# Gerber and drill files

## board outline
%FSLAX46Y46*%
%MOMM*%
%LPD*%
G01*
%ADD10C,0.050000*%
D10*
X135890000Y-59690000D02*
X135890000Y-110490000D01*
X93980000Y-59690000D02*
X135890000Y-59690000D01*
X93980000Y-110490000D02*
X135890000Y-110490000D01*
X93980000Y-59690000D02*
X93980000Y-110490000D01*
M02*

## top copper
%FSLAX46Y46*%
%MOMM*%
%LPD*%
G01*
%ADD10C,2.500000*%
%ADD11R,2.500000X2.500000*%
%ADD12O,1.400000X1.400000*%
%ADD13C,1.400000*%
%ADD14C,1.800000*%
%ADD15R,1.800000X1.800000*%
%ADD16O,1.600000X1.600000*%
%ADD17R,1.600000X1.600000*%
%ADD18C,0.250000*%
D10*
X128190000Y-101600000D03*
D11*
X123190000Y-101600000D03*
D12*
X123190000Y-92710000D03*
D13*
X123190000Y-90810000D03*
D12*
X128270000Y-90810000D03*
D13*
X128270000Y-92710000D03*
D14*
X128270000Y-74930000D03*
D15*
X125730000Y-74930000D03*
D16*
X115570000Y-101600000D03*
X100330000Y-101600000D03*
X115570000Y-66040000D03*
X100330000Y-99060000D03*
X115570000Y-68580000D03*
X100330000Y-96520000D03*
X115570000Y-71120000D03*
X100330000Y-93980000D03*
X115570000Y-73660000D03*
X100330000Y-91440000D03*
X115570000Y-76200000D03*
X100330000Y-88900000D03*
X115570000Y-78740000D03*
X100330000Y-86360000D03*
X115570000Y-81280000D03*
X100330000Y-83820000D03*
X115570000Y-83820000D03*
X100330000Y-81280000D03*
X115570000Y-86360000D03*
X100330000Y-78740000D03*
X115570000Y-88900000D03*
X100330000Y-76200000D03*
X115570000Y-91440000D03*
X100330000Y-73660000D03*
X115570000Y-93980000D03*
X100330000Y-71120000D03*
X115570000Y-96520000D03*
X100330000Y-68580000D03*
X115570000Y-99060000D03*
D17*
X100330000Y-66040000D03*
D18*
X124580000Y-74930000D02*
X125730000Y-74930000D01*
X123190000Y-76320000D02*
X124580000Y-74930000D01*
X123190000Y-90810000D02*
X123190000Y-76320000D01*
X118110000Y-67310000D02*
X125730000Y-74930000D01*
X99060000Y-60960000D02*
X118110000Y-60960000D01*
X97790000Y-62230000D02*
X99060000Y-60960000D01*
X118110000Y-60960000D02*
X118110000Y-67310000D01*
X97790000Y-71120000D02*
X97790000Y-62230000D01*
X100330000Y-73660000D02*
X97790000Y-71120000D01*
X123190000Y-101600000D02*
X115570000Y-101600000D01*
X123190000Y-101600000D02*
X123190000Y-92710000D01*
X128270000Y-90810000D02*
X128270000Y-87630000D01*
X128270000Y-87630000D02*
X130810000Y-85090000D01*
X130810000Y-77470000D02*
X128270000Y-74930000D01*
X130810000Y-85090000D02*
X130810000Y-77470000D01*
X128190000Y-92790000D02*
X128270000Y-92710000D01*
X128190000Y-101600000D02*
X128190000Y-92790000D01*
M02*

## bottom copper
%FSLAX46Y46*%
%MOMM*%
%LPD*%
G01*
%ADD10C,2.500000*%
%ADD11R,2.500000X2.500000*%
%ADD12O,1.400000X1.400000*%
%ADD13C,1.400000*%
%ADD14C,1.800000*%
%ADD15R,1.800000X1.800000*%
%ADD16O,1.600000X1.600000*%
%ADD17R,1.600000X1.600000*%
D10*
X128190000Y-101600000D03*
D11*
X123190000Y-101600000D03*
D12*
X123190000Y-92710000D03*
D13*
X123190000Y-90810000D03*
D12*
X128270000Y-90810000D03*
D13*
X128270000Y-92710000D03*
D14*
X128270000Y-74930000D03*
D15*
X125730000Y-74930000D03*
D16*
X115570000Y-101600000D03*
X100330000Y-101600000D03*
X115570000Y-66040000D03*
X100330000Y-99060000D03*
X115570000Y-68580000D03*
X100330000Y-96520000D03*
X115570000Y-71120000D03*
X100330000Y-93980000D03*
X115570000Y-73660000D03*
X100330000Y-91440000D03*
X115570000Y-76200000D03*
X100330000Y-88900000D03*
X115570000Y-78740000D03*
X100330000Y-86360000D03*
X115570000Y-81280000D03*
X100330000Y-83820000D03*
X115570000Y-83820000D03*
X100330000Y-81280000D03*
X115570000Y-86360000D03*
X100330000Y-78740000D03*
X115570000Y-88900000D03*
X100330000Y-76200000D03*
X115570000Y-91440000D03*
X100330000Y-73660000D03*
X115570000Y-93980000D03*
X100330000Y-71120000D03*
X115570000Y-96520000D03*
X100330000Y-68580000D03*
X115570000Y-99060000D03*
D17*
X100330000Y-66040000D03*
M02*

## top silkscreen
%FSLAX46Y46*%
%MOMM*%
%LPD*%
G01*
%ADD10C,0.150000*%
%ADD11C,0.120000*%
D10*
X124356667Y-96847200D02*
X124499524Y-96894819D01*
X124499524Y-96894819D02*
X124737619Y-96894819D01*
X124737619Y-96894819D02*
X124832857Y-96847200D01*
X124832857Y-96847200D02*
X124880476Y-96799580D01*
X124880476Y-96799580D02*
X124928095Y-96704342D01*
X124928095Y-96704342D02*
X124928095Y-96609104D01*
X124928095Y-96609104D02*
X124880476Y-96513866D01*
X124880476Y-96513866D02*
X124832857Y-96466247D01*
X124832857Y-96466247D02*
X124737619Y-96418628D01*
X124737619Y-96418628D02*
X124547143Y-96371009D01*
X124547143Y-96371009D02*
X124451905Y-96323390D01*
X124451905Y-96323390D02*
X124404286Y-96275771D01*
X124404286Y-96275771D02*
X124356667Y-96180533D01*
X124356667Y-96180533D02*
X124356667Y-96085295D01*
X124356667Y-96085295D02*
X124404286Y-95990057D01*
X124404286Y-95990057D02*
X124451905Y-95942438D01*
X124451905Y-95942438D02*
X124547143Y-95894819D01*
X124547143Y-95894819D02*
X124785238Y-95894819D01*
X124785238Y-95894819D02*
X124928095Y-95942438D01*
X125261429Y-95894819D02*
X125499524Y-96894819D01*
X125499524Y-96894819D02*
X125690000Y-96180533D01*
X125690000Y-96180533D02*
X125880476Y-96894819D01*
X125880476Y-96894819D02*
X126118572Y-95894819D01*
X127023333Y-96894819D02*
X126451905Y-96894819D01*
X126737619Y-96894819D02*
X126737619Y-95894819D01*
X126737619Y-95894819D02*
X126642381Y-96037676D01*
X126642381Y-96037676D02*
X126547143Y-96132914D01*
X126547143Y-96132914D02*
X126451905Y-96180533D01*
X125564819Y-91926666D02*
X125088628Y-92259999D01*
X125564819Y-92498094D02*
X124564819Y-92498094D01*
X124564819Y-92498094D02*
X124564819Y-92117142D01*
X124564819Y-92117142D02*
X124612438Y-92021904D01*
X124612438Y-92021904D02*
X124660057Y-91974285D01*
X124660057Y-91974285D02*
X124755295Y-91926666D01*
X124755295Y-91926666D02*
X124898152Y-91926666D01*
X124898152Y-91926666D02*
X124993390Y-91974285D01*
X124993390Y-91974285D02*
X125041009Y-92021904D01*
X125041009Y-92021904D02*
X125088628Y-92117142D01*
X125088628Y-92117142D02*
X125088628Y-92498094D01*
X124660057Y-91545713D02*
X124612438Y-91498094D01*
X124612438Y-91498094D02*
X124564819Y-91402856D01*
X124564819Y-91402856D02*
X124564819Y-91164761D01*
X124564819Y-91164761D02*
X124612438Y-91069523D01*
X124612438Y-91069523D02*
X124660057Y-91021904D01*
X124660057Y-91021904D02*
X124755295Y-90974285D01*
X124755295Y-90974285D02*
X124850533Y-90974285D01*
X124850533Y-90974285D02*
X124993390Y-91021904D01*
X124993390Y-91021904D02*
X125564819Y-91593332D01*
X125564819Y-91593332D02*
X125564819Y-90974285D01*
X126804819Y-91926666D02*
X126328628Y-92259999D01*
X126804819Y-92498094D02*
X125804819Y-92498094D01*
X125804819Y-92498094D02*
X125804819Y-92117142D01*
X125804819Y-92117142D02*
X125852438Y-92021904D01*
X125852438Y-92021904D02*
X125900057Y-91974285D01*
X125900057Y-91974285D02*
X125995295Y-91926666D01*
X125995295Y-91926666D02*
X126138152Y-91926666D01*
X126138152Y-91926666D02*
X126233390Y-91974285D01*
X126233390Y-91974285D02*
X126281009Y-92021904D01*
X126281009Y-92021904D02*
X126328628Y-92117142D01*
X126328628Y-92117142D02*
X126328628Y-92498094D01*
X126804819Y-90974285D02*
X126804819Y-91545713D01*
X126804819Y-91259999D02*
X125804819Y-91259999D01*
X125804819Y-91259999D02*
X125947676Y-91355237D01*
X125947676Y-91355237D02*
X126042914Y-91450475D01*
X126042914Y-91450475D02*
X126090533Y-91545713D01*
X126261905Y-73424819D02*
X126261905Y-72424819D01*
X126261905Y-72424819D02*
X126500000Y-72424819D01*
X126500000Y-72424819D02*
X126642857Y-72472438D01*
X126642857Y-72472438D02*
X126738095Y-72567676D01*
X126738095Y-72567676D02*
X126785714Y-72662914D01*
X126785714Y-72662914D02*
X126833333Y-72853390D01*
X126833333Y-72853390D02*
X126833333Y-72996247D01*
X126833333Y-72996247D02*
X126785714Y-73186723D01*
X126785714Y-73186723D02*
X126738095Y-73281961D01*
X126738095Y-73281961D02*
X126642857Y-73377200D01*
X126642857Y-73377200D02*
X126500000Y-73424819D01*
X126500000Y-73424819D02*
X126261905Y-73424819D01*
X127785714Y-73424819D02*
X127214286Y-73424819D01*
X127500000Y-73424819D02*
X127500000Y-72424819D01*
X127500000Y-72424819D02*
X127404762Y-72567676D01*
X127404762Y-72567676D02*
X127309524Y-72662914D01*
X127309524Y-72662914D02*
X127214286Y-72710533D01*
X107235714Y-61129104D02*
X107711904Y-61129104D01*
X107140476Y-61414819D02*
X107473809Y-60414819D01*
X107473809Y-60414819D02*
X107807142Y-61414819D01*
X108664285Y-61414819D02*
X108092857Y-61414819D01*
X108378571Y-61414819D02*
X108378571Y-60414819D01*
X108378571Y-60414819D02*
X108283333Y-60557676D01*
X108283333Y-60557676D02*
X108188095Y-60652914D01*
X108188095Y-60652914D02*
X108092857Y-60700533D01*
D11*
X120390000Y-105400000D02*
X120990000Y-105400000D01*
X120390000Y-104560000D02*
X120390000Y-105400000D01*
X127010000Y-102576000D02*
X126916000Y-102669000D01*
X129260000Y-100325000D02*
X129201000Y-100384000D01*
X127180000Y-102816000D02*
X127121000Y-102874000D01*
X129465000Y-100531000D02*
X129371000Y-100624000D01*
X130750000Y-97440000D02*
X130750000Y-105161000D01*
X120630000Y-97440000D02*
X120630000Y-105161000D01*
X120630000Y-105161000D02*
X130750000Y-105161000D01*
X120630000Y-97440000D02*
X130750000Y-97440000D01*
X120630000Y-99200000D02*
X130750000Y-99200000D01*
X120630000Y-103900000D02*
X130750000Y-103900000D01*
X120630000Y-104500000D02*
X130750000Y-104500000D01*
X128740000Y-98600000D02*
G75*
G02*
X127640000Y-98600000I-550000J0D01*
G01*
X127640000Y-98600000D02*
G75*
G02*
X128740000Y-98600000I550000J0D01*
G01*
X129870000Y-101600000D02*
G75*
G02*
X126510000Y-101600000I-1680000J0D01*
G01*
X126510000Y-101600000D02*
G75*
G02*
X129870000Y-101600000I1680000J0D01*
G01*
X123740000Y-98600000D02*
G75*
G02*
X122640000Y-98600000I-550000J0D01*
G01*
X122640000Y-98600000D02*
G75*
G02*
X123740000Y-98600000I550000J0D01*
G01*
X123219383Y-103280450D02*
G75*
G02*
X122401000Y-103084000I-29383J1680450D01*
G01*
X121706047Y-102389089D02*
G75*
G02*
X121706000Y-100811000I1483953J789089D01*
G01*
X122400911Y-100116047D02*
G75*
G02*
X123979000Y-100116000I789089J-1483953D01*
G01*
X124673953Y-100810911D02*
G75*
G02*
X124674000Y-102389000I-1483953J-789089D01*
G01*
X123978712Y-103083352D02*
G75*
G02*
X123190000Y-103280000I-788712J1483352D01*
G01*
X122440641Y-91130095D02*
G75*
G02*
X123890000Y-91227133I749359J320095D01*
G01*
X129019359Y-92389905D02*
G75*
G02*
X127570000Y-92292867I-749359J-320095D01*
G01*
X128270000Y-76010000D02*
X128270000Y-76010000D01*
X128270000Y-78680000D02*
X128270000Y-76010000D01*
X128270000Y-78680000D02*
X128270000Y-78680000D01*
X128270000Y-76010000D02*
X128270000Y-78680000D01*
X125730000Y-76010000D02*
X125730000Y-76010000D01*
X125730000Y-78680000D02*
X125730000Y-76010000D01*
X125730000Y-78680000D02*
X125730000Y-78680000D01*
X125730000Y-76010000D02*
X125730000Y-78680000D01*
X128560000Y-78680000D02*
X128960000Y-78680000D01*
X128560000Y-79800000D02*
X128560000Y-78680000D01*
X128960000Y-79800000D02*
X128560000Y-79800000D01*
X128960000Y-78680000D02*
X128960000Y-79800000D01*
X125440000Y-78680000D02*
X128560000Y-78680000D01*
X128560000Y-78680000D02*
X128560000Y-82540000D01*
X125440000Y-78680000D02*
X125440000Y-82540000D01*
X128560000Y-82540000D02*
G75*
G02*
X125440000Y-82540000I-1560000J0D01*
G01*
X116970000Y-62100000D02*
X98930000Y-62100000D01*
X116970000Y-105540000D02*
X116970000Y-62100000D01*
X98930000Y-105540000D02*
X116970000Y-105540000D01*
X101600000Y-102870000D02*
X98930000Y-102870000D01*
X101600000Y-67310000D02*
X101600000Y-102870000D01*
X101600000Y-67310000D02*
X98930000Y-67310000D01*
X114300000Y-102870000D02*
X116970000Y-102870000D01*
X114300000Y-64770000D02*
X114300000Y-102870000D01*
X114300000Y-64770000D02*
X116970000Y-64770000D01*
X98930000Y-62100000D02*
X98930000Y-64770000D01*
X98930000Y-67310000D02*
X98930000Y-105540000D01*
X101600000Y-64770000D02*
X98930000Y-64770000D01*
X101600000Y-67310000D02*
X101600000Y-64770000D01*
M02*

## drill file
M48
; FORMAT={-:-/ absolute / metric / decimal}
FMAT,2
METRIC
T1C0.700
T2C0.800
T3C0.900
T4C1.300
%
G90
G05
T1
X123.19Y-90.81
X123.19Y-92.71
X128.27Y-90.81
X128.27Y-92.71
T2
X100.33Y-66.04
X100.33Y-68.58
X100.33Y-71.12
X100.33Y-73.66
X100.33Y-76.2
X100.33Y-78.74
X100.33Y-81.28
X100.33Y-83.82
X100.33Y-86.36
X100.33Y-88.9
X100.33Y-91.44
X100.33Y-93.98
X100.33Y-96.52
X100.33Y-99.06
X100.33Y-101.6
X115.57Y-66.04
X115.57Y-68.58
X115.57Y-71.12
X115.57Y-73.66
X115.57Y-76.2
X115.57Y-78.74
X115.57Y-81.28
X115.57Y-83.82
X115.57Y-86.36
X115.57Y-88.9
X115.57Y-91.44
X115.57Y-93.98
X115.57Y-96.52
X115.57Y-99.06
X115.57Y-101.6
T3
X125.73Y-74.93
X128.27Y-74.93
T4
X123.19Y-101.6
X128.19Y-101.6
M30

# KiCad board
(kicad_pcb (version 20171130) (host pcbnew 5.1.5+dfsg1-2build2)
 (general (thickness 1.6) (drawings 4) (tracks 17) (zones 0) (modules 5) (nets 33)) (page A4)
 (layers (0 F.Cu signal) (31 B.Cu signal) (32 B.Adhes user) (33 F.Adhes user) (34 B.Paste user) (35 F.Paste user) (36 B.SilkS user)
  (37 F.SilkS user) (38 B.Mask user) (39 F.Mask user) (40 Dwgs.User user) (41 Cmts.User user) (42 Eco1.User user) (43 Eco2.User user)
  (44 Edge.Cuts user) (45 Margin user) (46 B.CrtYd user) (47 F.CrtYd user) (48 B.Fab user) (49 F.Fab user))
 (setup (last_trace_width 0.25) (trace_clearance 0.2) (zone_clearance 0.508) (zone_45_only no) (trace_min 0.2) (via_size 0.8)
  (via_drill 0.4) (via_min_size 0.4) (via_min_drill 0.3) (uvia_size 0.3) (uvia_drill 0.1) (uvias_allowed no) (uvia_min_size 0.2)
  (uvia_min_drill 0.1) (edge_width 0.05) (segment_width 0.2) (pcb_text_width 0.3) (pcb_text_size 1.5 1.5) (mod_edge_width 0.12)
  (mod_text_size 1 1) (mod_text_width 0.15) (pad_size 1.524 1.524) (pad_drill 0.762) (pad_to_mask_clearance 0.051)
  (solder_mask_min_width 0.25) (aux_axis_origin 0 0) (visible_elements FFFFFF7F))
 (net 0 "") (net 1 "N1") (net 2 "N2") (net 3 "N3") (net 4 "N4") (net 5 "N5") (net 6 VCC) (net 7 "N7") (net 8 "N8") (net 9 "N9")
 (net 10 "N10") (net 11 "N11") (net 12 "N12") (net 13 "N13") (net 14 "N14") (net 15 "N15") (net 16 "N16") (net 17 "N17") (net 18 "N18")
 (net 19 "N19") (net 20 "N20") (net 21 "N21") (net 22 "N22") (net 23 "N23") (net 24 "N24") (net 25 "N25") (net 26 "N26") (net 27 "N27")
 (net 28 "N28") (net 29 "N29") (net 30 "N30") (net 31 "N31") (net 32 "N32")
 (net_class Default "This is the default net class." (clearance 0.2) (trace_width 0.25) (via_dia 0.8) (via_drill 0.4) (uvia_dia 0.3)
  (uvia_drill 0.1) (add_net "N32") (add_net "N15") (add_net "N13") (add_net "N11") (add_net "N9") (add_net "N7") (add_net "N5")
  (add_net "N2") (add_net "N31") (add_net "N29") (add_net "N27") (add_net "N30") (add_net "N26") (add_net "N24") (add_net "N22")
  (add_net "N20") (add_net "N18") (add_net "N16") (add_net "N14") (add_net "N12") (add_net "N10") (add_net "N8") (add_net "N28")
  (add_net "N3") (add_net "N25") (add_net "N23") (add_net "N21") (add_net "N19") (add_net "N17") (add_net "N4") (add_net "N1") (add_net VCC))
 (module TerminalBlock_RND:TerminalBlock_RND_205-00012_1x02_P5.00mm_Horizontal (layer F.Cu) (at 123.19 101.6)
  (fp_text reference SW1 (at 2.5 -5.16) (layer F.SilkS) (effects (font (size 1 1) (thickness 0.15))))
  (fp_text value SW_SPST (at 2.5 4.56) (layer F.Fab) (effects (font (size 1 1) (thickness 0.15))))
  (fp_line (start -2.8 3.8) (end -2.2 3.8) (layer F.SilkS) (width 0.12))
  (fp_line (start -2.8 2.96) (end -2.8 3.8) (layer F.SilkS) (width 0.12))
  (fp_line (start 3.82 0.976) (end 3.726 1.069) (layer F.SilkS) (width 0.12))
  (fp_line (start 6.07 -1.275) (end 6.011 -1.216) (layer F.SilkS) (width 0.12))
  (fp_line (start 3.99 1.216) (end 3.931 1.274) (layer F.SilkS) (width 0.12))
  (fp_line (start 6.275 -1.069) (end 6.181 -0.976) (layer F.SilkS) (width 0.12))
  (fp_line (start 7.56 -4.16) (end 7.56 3.561) (layer F.SilkS) (width 0.12))
  (fp_line (start -2.56 -4.16) (end -2.56 3.561) (layer F.SilkS) (width 0.12))
  (fp_line (start -2.56 3.561) (end 7.56 3.561) (layer F.SilkS) (width 0.12))
  (fp_line (start -2.56 -4.16) (end 7.56 -4.16) (layer F.SilkS) (width 0.12))
  (fp_line (start -2.56 -2.4) (end 7.56 -2.4) (layer F.SilkS) (width 0.12))
  (fp_line (start -2.56 2.3) (end 7.56 2.3) (layer F.SilkS) (width 0.12))
  (fp_line (start -2.56 2.9) (end 7.56 2.9) (layer F.SilkS) (width 0.12))
  (fp_circle (center 5 -3) (end 5.55 -3) (layer F.SilkS) (width 0.12))
  (fp_circle (center 5 0) (end 6.68 0) (layer F.SilkS) (width 0.12))
  (fp_circle (center 0 -3) (end 0.55 -3) (layer F.SilkS) (width 0.12))
  (fp_arc (start 0 0) (end -0.789 1.484) (angle -29) (layer F.SilkS) (width 0.12))
  (fp_arc (start 0 0) (end -1.484 -0.789) (angle -56) (layer F.SilkS) (width 0.12))
  (fp_arc (start 0 0) (end 0.789 -1.484) (angle -56) (layer F.SilkS) (width 0.12))
  (fp_arc (start 0 0) (end 1.484 0.789) (angle -56) (layer F.SilkS) (width 0.12))
  (fp_arc (start 0 0) (end 0 1.68) (angle -28) (layer F.SilkS) (width 0.12))
  (pad 2 thru_hole circle (at 5 0) (size 2.5 2.5) (drill 1.3) (layers *.Cu *.Mask) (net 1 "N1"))
  (pad 1 thru_hole rect (at 0 0) (size 2.5 2.5) (drill 1.3) (layers *.Cu *.Mask) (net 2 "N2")))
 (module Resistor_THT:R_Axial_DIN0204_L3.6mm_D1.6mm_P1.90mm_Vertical (layer F.Cu) (at 123.19 90.81 270)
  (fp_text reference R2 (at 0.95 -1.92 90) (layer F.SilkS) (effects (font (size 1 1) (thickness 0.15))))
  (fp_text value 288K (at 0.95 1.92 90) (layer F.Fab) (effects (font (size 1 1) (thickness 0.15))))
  (fp_arc (start 0 0) (end 0.417133 -0.7) (angle -233.92106) (layer F.SilkS) (width 0.12))
  (pad 2 thru_hole oval (at 1.9 0 270) (size 1.4 1.4) (drill 0.7) (layers *.Cu *.Mask) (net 2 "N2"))
  (pad 1 thru_hole circle (at 0 0 270) (size 1.4 1.4) (drill 0.7) (layers *.Cu *.Mask) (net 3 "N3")))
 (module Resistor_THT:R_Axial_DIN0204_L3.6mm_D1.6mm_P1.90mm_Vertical (layer F.Cu) (at 128.27 92.71 90)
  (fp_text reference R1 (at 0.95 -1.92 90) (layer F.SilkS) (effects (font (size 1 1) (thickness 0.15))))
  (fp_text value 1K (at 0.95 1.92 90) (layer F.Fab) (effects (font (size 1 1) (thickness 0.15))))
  (fp_arc (start 0 0) (end 0.417133 -0.7) (angle -233.92106) (layer F.SilkS) (width 0.12))
  (pad 2 thru_hole oval (at 1.9 0 90) (size 1.4 1.4) (drill 0.7) (layers *.Cu *.Mask) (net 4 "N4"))
  (pad 1 thru_hole circle (at 0 0 90) (size 1.4 1.4) (drill 0.7) (layers *.Cu *.Mask) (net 1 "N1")))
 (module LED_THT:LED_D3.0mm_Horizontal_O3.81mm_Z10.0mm (layer F.Cu) (at 125.73 74.93)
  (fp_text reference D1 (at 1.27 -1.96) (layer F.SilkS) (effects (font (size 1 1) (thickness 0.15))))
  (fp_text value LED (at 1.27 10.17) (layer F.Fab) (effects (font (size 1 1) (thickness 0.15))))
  (fp_line (start 2.54 1.08) (end 2.54 1.08) (layer F.SilkS) (width 0.12))
  (fp_line (start 2.54 3.75) (end 2.54 1.08) (layer F.SilkS) (width 0.12))
  (fp_line (start 2.54 3.75) (end 2.54 3.75) (layer F.SilkS) (width 0.12))
  (fp_line (start 2.54 1.08) (end 2.54 3.75) (layer F.SilkS) (width 0.12))
  (fp_line (start 0 1.08) (end 0 1.08) (layer F.SilkS) (width 0.12))
  (fp_line (start 0 3.75) (end 0 1.08) (layer F.SilkS) (width 0.12))
  (fp_line (start 0 3.75) (end 0 3.75) (layer F.SilkS) (width 0.12))
  (fp_line (start 0 1.08) (end 0 3.75) (layer F.SilkS) (width 0.12))
  (fp_line (start 2.83 3.75) (end 3.23 3.75) (layer F.SilkS) (width 0.12))
  (fp_line (start 2.83 4.87) (end 2.83 3.75) (layer F.SilkS) (width 0.12))
  (fp_line (start 3.23 4.87) (end 2.83 4.87) (layer F.SilkS) (width 0.12))
  (fp_line (start 3.23 3.75) (end 3.23 4.87) (layer F.SilkS) (width 0.12))
  (fp_line (start -0.29 3.75) (end 2.83 3.75) (layer F.SilkS) (width 0.12))
  (fp_line (start 2.83 3.75) (end 2.83 7.61) (layer F.SilkS) (width 0.12))
  (fp_line (start -0.29 3.75) (end -0.29 7.61) (layer F.SilkS) (width 0.12))
  (fp_arc (start 1.27 7.61) (end -0.29 7.61) (angle -180) (layer F.SilkS) (width 0.12))
  (pad 2 thru_hole circle (at 2.54 0) (size 1.8 1.8) (drill 0.9) (layers *.Cu *.Mask) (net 4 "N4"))
  (pad 1 thru_hole rect (at 0 0) (size 1.8 1.8) (drill 0.9) (layers *.Cu *.Mask) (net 3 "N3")))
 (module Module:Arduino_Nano (layer F.Cu) (at 100.33 66.04)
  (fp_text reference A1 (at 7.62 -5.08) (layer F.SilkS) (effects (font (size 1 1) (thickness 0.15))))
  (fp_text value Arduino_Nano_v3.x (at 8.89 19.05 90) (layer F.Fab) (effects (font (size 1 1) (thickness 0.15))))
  (fp_line (start 16.64 -3.94) (end -1.4 -3.94) (layer F.SilkS) (width 0.12))
  (fp_line (start 16.64 39.5) (end 16.64 -3.94) (layer F.SilkS) (width 0.12))
  (fp_line (start -1.4 39.5) (end 16.64 39.5) (layer F.SilkS) (width 0.12))
  (fp_line (start 1.27 36.83) (end -1.4 36.83) (layer F.SilkS) (width 0.12))
  (fp_line (start 1.27 1.27) (end 1.27 36.83) (layer F.SilkS) (width 0.12))
  (fp_line (start 1.27 1.27) (end -1.4 1.27) (layer F.SilkS) (width 0.12))
  (fp_line (start 13.97 36.83) (end 16.64 36.83) (layer F.SilkS) (width 0.12))
  (fp_line (start 13.97 -1.27) (end 13.97 36.83) (layer F.SilkS) (width 0.12))
  (fp_line (start 13.97 -1.27) (end 16.64 -1.27) (layer F.SilkS) (width 0.12))
  (fp_line (start -1.4 -3.94) (end -1.4 -1.27) (layer F.SilkS) (width 0.12))
  (fp_line (start -1.4 1.27) (end -1.4 39.5) (layer F.SilkS) (width 0.12))
  (fp_line (start 1.27 -1.27) (end -1.4 -1.27) (layer F.SilkS) (width 0.12))
  (fp_line (start 1.27 1.27) (end 1.27 -1.27) (layer F.SilkS) (width 0.12))
  (pad 16 thru_hole oval (at 15.24 35.56) (size 1.6 1.6) (drill 0.8) (layers *.Cu *.Mask) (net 2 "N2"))
  (pad 15 thru_hole oval (at 0 35.56) (size 1.6 1.6) (drill 0.8) (layers *.Cu *.Mask) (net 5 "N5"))
  (pad 30 thru_hole oval (at 15.24 0) (size 1.6 1.6) (drill 0.8) (layers *.Cu *.Mask) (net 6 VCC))
  (pad 14 thru_hole oval (at 0 33.02) (size 1.6 1.6) (drill 0.8) (layers *.Cu *.Mask) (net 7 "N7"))
  (pad 29 thru_hole oval (at 15.24 2.54) (size 1.6 1.6) (drill 0.8) (layers *.Cu *.Mask) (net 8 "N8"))
  (pad 13 thru_hole oval (at 0 30.48) (size 1.6 1.6) (drill 0.8) (layers *.Cu *.Mask) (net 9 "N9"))
  (pad 28 thru_hole oval (at 15.24 5.08) (size 1.6 1.6) (drill 0.8) (layers *.Cu *.Mask) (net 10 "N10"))
  (pad 12 thru_hole oval (at 0 27.94) (size 1.6 1.6) (drill 0.8) (layers *.Cu *.Mask) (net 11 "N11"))
  (pad 27 thru_hole oval (at 15.24 7.62) (size 1.6 1.6) (drill 0.8) (layers *.Cu *.Mask) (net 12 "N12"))
  (pad 11 thru_hole oval (at 0 25.4) (size 1.6 1.6) (drill 0.8) (layers *.Cu *.Mask) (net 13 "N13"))
  (pad 26 thru_hole oval (at 15.24 10.16) (size 1.6 1.6) (drill 0.8) (layers *.Cu *.Mask) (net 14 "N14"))
  (pad 10 thru_hole oval (at 0 22.86) (size 1.6 1.6) (drill 0.8) (layers *.Cu *.Mask) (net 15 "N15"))
  (pad 25 thru_hole oval (at 15.24 12.7) (size 1.6 1.6) (drill 0.8) (layers *.Cu *.Mask) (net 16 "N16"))
  (pad 9 thru_hole oval (at 0 20.32) (size 1.6 1.6) (drill 0.8) (layers *.Cu *.Mask) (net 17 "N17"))
  (pad 24 thru_hole oval (at 15.24 15.24) (size 1.6 1.6) (drill 0.8) (layers *.Cu *.Mask) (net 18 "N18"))
  (pad 8 thru_hole oval (at 0 17.78) (size 1.6 1.6) (drill 0.8) (layers *.Cu *.Mask) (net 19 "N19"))
  (pad 23 thru_hole oval (at 15.24 17.78) (size 1.6 1.6) (drill 0.8) (layers *.Cu *.Mask) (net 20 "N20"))
  (pad 7 thru_hole oval (at 0 15.24) (size 1.6 1.6) (drill 0.8) (layers *.Cu *.Mask) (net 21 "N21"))
  (pad 22 thru_hole oval (at 15.24 20.32) (size 1.6 1.6) (drill 0.8) (layers *.Cu *.Mask) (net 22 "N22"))
  (pad 6 thru_hole oval (at 0 12.7) (size 1.6 1.6) (drill 0.8) (layers *.Cu *.Mask) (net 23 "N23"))
  (pad 21 thru_hole oval (at 15.24 22.86) (size 1.6 1.6) (drill 0.8) (layers *.Cu *.Mask) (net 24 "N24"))
  (pad 5 thru_hole oval (at 0 10.16) (size 1.6 1.6) (drill 0.8) (layers *.Cu *.Mask) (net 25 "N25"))
  (pad 20 thru_hole oval (at 15.24 25.4) (size 1.6 1.6) (drill 0.8) (layers *.Cu *.Mask) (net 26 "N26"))
  (pad 4 thru_hole oval (at 0 7.62) (size 1.6 1.6) (drill 0.8) (layers *.Cu *.Mask) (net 3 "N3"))
  (pad 19 thru_hole oval (at 15.24 27.94) (size 1.6 1.6) (drill 0.8) (layers *.Cu *.Mask) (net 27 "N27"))
  (pad 3 thru_hole oval (at 0 5.08) (size 1.6 1.6) (drill 0.8) (layers *.Cu *.Mask) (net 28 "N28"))
  (pad 18 thru_hole oval (at 15.24 30.48) (size 1.6 1.6) (drill 0.8) (layers *.Cu *.Mask) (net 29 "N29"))
  (pad 2 thru_hole oval (at 0 2.54) (size 1.6 1.6) (drill 0.8) (layers *.Cu *.Mask) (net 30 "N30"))
  (pad 17 thru_hole oval (at 15.24 33.02) (size 1.6 1.6) (drill 0.8) (layers *.Cu *.Mask) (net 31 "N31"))
  (pad 1 thru_hole rect (at 0 0) (size 1.6 1.6) (drill 0.8) (layers *.Cu *.Mask) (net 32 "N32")))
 (gr_line (start 135.89 59.69) (end 135.89 110.49) (layer Edge.Cuts) (width 0.05))
 (gr_line (start 93.98 59.69) (end 135.89 59.69) (layer Edge.Cuts) (width 0.05))
 (gr_line (start 93.98 110.49) (end 135.89 110.49) (layer Edge.Cuts) (width 0.05))
 (gr_line (start 93.98 59.69) (end 93.98 110.49) (layer Edge.Cuts) (width 0.05))
 (segment (start 124.58 74.93) (end 125.73 74.93) (width 0.25) (layer F.Cu) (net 3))
 (segment (start 123.19 76.32) (end 124.58 74.93) (width 0.25) (layer F.Cu) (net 3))
 (segment (start 123.19 90.81) (end 123.19 76.32) (width 0.25) (layer F.Cu) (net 3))
 (segment (start 118.11 67.31) (end 125.73 74.93) (width 0.25) (layer F.Cu) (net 3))
 (segment (start 99.06 60.96) (end 118.11 60.96) (width 0.25) (layer F.Cu) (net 3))
 (segment (start 97.79 62.23) (end 99.06 60.96) (width 0.25) (layer F.Cu) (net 3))
 (segment (start 118.11 60.96) (end 118.11 67.31) (width 0.25) (layer F.Cu) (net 3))
 (segment (start 97.79 71.12) (end 97.79 62.23) (width 0.25) (layer F.Cu) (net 3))
 (segment (start 100.33 73.66) (end 97.79 71.12) (width 0.25) (layer F.Cu) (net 3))
 (segment (start 123.19 101.6) (end 115.57 101.6) (width 0.25) (layer F.Cu) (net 2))
 (segment (start 123.19 101.6) (end 123.19 92.71) (width 0.25) (layer F.Cu) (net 2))
 (segment (start 128.27 90.81) (end 128.27 87.63) (width 0.25) (layer F.Cu) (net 4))
 (segment (start 128.27 87.63) (end 130.81 85.09) (width 0.25) (layer F.Cu) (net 4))
 (segment (start 130.81 77.47) (end 128.27 74.93) (width 0.25) (layer F.Cu) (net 4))
 (segment (start 130.81 85.09) (end 130.81 77.47) (width 0.25) (layer F.Cu) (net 4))
 (segment (start 128.19 92.79) (end 128.27 92.71) (width 0.25) (layer F.Cu) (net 1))
 (segment (start 128.19 101.6) (end 128.19 92.79) (width 0.25) (layer F.Cu) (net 1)))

